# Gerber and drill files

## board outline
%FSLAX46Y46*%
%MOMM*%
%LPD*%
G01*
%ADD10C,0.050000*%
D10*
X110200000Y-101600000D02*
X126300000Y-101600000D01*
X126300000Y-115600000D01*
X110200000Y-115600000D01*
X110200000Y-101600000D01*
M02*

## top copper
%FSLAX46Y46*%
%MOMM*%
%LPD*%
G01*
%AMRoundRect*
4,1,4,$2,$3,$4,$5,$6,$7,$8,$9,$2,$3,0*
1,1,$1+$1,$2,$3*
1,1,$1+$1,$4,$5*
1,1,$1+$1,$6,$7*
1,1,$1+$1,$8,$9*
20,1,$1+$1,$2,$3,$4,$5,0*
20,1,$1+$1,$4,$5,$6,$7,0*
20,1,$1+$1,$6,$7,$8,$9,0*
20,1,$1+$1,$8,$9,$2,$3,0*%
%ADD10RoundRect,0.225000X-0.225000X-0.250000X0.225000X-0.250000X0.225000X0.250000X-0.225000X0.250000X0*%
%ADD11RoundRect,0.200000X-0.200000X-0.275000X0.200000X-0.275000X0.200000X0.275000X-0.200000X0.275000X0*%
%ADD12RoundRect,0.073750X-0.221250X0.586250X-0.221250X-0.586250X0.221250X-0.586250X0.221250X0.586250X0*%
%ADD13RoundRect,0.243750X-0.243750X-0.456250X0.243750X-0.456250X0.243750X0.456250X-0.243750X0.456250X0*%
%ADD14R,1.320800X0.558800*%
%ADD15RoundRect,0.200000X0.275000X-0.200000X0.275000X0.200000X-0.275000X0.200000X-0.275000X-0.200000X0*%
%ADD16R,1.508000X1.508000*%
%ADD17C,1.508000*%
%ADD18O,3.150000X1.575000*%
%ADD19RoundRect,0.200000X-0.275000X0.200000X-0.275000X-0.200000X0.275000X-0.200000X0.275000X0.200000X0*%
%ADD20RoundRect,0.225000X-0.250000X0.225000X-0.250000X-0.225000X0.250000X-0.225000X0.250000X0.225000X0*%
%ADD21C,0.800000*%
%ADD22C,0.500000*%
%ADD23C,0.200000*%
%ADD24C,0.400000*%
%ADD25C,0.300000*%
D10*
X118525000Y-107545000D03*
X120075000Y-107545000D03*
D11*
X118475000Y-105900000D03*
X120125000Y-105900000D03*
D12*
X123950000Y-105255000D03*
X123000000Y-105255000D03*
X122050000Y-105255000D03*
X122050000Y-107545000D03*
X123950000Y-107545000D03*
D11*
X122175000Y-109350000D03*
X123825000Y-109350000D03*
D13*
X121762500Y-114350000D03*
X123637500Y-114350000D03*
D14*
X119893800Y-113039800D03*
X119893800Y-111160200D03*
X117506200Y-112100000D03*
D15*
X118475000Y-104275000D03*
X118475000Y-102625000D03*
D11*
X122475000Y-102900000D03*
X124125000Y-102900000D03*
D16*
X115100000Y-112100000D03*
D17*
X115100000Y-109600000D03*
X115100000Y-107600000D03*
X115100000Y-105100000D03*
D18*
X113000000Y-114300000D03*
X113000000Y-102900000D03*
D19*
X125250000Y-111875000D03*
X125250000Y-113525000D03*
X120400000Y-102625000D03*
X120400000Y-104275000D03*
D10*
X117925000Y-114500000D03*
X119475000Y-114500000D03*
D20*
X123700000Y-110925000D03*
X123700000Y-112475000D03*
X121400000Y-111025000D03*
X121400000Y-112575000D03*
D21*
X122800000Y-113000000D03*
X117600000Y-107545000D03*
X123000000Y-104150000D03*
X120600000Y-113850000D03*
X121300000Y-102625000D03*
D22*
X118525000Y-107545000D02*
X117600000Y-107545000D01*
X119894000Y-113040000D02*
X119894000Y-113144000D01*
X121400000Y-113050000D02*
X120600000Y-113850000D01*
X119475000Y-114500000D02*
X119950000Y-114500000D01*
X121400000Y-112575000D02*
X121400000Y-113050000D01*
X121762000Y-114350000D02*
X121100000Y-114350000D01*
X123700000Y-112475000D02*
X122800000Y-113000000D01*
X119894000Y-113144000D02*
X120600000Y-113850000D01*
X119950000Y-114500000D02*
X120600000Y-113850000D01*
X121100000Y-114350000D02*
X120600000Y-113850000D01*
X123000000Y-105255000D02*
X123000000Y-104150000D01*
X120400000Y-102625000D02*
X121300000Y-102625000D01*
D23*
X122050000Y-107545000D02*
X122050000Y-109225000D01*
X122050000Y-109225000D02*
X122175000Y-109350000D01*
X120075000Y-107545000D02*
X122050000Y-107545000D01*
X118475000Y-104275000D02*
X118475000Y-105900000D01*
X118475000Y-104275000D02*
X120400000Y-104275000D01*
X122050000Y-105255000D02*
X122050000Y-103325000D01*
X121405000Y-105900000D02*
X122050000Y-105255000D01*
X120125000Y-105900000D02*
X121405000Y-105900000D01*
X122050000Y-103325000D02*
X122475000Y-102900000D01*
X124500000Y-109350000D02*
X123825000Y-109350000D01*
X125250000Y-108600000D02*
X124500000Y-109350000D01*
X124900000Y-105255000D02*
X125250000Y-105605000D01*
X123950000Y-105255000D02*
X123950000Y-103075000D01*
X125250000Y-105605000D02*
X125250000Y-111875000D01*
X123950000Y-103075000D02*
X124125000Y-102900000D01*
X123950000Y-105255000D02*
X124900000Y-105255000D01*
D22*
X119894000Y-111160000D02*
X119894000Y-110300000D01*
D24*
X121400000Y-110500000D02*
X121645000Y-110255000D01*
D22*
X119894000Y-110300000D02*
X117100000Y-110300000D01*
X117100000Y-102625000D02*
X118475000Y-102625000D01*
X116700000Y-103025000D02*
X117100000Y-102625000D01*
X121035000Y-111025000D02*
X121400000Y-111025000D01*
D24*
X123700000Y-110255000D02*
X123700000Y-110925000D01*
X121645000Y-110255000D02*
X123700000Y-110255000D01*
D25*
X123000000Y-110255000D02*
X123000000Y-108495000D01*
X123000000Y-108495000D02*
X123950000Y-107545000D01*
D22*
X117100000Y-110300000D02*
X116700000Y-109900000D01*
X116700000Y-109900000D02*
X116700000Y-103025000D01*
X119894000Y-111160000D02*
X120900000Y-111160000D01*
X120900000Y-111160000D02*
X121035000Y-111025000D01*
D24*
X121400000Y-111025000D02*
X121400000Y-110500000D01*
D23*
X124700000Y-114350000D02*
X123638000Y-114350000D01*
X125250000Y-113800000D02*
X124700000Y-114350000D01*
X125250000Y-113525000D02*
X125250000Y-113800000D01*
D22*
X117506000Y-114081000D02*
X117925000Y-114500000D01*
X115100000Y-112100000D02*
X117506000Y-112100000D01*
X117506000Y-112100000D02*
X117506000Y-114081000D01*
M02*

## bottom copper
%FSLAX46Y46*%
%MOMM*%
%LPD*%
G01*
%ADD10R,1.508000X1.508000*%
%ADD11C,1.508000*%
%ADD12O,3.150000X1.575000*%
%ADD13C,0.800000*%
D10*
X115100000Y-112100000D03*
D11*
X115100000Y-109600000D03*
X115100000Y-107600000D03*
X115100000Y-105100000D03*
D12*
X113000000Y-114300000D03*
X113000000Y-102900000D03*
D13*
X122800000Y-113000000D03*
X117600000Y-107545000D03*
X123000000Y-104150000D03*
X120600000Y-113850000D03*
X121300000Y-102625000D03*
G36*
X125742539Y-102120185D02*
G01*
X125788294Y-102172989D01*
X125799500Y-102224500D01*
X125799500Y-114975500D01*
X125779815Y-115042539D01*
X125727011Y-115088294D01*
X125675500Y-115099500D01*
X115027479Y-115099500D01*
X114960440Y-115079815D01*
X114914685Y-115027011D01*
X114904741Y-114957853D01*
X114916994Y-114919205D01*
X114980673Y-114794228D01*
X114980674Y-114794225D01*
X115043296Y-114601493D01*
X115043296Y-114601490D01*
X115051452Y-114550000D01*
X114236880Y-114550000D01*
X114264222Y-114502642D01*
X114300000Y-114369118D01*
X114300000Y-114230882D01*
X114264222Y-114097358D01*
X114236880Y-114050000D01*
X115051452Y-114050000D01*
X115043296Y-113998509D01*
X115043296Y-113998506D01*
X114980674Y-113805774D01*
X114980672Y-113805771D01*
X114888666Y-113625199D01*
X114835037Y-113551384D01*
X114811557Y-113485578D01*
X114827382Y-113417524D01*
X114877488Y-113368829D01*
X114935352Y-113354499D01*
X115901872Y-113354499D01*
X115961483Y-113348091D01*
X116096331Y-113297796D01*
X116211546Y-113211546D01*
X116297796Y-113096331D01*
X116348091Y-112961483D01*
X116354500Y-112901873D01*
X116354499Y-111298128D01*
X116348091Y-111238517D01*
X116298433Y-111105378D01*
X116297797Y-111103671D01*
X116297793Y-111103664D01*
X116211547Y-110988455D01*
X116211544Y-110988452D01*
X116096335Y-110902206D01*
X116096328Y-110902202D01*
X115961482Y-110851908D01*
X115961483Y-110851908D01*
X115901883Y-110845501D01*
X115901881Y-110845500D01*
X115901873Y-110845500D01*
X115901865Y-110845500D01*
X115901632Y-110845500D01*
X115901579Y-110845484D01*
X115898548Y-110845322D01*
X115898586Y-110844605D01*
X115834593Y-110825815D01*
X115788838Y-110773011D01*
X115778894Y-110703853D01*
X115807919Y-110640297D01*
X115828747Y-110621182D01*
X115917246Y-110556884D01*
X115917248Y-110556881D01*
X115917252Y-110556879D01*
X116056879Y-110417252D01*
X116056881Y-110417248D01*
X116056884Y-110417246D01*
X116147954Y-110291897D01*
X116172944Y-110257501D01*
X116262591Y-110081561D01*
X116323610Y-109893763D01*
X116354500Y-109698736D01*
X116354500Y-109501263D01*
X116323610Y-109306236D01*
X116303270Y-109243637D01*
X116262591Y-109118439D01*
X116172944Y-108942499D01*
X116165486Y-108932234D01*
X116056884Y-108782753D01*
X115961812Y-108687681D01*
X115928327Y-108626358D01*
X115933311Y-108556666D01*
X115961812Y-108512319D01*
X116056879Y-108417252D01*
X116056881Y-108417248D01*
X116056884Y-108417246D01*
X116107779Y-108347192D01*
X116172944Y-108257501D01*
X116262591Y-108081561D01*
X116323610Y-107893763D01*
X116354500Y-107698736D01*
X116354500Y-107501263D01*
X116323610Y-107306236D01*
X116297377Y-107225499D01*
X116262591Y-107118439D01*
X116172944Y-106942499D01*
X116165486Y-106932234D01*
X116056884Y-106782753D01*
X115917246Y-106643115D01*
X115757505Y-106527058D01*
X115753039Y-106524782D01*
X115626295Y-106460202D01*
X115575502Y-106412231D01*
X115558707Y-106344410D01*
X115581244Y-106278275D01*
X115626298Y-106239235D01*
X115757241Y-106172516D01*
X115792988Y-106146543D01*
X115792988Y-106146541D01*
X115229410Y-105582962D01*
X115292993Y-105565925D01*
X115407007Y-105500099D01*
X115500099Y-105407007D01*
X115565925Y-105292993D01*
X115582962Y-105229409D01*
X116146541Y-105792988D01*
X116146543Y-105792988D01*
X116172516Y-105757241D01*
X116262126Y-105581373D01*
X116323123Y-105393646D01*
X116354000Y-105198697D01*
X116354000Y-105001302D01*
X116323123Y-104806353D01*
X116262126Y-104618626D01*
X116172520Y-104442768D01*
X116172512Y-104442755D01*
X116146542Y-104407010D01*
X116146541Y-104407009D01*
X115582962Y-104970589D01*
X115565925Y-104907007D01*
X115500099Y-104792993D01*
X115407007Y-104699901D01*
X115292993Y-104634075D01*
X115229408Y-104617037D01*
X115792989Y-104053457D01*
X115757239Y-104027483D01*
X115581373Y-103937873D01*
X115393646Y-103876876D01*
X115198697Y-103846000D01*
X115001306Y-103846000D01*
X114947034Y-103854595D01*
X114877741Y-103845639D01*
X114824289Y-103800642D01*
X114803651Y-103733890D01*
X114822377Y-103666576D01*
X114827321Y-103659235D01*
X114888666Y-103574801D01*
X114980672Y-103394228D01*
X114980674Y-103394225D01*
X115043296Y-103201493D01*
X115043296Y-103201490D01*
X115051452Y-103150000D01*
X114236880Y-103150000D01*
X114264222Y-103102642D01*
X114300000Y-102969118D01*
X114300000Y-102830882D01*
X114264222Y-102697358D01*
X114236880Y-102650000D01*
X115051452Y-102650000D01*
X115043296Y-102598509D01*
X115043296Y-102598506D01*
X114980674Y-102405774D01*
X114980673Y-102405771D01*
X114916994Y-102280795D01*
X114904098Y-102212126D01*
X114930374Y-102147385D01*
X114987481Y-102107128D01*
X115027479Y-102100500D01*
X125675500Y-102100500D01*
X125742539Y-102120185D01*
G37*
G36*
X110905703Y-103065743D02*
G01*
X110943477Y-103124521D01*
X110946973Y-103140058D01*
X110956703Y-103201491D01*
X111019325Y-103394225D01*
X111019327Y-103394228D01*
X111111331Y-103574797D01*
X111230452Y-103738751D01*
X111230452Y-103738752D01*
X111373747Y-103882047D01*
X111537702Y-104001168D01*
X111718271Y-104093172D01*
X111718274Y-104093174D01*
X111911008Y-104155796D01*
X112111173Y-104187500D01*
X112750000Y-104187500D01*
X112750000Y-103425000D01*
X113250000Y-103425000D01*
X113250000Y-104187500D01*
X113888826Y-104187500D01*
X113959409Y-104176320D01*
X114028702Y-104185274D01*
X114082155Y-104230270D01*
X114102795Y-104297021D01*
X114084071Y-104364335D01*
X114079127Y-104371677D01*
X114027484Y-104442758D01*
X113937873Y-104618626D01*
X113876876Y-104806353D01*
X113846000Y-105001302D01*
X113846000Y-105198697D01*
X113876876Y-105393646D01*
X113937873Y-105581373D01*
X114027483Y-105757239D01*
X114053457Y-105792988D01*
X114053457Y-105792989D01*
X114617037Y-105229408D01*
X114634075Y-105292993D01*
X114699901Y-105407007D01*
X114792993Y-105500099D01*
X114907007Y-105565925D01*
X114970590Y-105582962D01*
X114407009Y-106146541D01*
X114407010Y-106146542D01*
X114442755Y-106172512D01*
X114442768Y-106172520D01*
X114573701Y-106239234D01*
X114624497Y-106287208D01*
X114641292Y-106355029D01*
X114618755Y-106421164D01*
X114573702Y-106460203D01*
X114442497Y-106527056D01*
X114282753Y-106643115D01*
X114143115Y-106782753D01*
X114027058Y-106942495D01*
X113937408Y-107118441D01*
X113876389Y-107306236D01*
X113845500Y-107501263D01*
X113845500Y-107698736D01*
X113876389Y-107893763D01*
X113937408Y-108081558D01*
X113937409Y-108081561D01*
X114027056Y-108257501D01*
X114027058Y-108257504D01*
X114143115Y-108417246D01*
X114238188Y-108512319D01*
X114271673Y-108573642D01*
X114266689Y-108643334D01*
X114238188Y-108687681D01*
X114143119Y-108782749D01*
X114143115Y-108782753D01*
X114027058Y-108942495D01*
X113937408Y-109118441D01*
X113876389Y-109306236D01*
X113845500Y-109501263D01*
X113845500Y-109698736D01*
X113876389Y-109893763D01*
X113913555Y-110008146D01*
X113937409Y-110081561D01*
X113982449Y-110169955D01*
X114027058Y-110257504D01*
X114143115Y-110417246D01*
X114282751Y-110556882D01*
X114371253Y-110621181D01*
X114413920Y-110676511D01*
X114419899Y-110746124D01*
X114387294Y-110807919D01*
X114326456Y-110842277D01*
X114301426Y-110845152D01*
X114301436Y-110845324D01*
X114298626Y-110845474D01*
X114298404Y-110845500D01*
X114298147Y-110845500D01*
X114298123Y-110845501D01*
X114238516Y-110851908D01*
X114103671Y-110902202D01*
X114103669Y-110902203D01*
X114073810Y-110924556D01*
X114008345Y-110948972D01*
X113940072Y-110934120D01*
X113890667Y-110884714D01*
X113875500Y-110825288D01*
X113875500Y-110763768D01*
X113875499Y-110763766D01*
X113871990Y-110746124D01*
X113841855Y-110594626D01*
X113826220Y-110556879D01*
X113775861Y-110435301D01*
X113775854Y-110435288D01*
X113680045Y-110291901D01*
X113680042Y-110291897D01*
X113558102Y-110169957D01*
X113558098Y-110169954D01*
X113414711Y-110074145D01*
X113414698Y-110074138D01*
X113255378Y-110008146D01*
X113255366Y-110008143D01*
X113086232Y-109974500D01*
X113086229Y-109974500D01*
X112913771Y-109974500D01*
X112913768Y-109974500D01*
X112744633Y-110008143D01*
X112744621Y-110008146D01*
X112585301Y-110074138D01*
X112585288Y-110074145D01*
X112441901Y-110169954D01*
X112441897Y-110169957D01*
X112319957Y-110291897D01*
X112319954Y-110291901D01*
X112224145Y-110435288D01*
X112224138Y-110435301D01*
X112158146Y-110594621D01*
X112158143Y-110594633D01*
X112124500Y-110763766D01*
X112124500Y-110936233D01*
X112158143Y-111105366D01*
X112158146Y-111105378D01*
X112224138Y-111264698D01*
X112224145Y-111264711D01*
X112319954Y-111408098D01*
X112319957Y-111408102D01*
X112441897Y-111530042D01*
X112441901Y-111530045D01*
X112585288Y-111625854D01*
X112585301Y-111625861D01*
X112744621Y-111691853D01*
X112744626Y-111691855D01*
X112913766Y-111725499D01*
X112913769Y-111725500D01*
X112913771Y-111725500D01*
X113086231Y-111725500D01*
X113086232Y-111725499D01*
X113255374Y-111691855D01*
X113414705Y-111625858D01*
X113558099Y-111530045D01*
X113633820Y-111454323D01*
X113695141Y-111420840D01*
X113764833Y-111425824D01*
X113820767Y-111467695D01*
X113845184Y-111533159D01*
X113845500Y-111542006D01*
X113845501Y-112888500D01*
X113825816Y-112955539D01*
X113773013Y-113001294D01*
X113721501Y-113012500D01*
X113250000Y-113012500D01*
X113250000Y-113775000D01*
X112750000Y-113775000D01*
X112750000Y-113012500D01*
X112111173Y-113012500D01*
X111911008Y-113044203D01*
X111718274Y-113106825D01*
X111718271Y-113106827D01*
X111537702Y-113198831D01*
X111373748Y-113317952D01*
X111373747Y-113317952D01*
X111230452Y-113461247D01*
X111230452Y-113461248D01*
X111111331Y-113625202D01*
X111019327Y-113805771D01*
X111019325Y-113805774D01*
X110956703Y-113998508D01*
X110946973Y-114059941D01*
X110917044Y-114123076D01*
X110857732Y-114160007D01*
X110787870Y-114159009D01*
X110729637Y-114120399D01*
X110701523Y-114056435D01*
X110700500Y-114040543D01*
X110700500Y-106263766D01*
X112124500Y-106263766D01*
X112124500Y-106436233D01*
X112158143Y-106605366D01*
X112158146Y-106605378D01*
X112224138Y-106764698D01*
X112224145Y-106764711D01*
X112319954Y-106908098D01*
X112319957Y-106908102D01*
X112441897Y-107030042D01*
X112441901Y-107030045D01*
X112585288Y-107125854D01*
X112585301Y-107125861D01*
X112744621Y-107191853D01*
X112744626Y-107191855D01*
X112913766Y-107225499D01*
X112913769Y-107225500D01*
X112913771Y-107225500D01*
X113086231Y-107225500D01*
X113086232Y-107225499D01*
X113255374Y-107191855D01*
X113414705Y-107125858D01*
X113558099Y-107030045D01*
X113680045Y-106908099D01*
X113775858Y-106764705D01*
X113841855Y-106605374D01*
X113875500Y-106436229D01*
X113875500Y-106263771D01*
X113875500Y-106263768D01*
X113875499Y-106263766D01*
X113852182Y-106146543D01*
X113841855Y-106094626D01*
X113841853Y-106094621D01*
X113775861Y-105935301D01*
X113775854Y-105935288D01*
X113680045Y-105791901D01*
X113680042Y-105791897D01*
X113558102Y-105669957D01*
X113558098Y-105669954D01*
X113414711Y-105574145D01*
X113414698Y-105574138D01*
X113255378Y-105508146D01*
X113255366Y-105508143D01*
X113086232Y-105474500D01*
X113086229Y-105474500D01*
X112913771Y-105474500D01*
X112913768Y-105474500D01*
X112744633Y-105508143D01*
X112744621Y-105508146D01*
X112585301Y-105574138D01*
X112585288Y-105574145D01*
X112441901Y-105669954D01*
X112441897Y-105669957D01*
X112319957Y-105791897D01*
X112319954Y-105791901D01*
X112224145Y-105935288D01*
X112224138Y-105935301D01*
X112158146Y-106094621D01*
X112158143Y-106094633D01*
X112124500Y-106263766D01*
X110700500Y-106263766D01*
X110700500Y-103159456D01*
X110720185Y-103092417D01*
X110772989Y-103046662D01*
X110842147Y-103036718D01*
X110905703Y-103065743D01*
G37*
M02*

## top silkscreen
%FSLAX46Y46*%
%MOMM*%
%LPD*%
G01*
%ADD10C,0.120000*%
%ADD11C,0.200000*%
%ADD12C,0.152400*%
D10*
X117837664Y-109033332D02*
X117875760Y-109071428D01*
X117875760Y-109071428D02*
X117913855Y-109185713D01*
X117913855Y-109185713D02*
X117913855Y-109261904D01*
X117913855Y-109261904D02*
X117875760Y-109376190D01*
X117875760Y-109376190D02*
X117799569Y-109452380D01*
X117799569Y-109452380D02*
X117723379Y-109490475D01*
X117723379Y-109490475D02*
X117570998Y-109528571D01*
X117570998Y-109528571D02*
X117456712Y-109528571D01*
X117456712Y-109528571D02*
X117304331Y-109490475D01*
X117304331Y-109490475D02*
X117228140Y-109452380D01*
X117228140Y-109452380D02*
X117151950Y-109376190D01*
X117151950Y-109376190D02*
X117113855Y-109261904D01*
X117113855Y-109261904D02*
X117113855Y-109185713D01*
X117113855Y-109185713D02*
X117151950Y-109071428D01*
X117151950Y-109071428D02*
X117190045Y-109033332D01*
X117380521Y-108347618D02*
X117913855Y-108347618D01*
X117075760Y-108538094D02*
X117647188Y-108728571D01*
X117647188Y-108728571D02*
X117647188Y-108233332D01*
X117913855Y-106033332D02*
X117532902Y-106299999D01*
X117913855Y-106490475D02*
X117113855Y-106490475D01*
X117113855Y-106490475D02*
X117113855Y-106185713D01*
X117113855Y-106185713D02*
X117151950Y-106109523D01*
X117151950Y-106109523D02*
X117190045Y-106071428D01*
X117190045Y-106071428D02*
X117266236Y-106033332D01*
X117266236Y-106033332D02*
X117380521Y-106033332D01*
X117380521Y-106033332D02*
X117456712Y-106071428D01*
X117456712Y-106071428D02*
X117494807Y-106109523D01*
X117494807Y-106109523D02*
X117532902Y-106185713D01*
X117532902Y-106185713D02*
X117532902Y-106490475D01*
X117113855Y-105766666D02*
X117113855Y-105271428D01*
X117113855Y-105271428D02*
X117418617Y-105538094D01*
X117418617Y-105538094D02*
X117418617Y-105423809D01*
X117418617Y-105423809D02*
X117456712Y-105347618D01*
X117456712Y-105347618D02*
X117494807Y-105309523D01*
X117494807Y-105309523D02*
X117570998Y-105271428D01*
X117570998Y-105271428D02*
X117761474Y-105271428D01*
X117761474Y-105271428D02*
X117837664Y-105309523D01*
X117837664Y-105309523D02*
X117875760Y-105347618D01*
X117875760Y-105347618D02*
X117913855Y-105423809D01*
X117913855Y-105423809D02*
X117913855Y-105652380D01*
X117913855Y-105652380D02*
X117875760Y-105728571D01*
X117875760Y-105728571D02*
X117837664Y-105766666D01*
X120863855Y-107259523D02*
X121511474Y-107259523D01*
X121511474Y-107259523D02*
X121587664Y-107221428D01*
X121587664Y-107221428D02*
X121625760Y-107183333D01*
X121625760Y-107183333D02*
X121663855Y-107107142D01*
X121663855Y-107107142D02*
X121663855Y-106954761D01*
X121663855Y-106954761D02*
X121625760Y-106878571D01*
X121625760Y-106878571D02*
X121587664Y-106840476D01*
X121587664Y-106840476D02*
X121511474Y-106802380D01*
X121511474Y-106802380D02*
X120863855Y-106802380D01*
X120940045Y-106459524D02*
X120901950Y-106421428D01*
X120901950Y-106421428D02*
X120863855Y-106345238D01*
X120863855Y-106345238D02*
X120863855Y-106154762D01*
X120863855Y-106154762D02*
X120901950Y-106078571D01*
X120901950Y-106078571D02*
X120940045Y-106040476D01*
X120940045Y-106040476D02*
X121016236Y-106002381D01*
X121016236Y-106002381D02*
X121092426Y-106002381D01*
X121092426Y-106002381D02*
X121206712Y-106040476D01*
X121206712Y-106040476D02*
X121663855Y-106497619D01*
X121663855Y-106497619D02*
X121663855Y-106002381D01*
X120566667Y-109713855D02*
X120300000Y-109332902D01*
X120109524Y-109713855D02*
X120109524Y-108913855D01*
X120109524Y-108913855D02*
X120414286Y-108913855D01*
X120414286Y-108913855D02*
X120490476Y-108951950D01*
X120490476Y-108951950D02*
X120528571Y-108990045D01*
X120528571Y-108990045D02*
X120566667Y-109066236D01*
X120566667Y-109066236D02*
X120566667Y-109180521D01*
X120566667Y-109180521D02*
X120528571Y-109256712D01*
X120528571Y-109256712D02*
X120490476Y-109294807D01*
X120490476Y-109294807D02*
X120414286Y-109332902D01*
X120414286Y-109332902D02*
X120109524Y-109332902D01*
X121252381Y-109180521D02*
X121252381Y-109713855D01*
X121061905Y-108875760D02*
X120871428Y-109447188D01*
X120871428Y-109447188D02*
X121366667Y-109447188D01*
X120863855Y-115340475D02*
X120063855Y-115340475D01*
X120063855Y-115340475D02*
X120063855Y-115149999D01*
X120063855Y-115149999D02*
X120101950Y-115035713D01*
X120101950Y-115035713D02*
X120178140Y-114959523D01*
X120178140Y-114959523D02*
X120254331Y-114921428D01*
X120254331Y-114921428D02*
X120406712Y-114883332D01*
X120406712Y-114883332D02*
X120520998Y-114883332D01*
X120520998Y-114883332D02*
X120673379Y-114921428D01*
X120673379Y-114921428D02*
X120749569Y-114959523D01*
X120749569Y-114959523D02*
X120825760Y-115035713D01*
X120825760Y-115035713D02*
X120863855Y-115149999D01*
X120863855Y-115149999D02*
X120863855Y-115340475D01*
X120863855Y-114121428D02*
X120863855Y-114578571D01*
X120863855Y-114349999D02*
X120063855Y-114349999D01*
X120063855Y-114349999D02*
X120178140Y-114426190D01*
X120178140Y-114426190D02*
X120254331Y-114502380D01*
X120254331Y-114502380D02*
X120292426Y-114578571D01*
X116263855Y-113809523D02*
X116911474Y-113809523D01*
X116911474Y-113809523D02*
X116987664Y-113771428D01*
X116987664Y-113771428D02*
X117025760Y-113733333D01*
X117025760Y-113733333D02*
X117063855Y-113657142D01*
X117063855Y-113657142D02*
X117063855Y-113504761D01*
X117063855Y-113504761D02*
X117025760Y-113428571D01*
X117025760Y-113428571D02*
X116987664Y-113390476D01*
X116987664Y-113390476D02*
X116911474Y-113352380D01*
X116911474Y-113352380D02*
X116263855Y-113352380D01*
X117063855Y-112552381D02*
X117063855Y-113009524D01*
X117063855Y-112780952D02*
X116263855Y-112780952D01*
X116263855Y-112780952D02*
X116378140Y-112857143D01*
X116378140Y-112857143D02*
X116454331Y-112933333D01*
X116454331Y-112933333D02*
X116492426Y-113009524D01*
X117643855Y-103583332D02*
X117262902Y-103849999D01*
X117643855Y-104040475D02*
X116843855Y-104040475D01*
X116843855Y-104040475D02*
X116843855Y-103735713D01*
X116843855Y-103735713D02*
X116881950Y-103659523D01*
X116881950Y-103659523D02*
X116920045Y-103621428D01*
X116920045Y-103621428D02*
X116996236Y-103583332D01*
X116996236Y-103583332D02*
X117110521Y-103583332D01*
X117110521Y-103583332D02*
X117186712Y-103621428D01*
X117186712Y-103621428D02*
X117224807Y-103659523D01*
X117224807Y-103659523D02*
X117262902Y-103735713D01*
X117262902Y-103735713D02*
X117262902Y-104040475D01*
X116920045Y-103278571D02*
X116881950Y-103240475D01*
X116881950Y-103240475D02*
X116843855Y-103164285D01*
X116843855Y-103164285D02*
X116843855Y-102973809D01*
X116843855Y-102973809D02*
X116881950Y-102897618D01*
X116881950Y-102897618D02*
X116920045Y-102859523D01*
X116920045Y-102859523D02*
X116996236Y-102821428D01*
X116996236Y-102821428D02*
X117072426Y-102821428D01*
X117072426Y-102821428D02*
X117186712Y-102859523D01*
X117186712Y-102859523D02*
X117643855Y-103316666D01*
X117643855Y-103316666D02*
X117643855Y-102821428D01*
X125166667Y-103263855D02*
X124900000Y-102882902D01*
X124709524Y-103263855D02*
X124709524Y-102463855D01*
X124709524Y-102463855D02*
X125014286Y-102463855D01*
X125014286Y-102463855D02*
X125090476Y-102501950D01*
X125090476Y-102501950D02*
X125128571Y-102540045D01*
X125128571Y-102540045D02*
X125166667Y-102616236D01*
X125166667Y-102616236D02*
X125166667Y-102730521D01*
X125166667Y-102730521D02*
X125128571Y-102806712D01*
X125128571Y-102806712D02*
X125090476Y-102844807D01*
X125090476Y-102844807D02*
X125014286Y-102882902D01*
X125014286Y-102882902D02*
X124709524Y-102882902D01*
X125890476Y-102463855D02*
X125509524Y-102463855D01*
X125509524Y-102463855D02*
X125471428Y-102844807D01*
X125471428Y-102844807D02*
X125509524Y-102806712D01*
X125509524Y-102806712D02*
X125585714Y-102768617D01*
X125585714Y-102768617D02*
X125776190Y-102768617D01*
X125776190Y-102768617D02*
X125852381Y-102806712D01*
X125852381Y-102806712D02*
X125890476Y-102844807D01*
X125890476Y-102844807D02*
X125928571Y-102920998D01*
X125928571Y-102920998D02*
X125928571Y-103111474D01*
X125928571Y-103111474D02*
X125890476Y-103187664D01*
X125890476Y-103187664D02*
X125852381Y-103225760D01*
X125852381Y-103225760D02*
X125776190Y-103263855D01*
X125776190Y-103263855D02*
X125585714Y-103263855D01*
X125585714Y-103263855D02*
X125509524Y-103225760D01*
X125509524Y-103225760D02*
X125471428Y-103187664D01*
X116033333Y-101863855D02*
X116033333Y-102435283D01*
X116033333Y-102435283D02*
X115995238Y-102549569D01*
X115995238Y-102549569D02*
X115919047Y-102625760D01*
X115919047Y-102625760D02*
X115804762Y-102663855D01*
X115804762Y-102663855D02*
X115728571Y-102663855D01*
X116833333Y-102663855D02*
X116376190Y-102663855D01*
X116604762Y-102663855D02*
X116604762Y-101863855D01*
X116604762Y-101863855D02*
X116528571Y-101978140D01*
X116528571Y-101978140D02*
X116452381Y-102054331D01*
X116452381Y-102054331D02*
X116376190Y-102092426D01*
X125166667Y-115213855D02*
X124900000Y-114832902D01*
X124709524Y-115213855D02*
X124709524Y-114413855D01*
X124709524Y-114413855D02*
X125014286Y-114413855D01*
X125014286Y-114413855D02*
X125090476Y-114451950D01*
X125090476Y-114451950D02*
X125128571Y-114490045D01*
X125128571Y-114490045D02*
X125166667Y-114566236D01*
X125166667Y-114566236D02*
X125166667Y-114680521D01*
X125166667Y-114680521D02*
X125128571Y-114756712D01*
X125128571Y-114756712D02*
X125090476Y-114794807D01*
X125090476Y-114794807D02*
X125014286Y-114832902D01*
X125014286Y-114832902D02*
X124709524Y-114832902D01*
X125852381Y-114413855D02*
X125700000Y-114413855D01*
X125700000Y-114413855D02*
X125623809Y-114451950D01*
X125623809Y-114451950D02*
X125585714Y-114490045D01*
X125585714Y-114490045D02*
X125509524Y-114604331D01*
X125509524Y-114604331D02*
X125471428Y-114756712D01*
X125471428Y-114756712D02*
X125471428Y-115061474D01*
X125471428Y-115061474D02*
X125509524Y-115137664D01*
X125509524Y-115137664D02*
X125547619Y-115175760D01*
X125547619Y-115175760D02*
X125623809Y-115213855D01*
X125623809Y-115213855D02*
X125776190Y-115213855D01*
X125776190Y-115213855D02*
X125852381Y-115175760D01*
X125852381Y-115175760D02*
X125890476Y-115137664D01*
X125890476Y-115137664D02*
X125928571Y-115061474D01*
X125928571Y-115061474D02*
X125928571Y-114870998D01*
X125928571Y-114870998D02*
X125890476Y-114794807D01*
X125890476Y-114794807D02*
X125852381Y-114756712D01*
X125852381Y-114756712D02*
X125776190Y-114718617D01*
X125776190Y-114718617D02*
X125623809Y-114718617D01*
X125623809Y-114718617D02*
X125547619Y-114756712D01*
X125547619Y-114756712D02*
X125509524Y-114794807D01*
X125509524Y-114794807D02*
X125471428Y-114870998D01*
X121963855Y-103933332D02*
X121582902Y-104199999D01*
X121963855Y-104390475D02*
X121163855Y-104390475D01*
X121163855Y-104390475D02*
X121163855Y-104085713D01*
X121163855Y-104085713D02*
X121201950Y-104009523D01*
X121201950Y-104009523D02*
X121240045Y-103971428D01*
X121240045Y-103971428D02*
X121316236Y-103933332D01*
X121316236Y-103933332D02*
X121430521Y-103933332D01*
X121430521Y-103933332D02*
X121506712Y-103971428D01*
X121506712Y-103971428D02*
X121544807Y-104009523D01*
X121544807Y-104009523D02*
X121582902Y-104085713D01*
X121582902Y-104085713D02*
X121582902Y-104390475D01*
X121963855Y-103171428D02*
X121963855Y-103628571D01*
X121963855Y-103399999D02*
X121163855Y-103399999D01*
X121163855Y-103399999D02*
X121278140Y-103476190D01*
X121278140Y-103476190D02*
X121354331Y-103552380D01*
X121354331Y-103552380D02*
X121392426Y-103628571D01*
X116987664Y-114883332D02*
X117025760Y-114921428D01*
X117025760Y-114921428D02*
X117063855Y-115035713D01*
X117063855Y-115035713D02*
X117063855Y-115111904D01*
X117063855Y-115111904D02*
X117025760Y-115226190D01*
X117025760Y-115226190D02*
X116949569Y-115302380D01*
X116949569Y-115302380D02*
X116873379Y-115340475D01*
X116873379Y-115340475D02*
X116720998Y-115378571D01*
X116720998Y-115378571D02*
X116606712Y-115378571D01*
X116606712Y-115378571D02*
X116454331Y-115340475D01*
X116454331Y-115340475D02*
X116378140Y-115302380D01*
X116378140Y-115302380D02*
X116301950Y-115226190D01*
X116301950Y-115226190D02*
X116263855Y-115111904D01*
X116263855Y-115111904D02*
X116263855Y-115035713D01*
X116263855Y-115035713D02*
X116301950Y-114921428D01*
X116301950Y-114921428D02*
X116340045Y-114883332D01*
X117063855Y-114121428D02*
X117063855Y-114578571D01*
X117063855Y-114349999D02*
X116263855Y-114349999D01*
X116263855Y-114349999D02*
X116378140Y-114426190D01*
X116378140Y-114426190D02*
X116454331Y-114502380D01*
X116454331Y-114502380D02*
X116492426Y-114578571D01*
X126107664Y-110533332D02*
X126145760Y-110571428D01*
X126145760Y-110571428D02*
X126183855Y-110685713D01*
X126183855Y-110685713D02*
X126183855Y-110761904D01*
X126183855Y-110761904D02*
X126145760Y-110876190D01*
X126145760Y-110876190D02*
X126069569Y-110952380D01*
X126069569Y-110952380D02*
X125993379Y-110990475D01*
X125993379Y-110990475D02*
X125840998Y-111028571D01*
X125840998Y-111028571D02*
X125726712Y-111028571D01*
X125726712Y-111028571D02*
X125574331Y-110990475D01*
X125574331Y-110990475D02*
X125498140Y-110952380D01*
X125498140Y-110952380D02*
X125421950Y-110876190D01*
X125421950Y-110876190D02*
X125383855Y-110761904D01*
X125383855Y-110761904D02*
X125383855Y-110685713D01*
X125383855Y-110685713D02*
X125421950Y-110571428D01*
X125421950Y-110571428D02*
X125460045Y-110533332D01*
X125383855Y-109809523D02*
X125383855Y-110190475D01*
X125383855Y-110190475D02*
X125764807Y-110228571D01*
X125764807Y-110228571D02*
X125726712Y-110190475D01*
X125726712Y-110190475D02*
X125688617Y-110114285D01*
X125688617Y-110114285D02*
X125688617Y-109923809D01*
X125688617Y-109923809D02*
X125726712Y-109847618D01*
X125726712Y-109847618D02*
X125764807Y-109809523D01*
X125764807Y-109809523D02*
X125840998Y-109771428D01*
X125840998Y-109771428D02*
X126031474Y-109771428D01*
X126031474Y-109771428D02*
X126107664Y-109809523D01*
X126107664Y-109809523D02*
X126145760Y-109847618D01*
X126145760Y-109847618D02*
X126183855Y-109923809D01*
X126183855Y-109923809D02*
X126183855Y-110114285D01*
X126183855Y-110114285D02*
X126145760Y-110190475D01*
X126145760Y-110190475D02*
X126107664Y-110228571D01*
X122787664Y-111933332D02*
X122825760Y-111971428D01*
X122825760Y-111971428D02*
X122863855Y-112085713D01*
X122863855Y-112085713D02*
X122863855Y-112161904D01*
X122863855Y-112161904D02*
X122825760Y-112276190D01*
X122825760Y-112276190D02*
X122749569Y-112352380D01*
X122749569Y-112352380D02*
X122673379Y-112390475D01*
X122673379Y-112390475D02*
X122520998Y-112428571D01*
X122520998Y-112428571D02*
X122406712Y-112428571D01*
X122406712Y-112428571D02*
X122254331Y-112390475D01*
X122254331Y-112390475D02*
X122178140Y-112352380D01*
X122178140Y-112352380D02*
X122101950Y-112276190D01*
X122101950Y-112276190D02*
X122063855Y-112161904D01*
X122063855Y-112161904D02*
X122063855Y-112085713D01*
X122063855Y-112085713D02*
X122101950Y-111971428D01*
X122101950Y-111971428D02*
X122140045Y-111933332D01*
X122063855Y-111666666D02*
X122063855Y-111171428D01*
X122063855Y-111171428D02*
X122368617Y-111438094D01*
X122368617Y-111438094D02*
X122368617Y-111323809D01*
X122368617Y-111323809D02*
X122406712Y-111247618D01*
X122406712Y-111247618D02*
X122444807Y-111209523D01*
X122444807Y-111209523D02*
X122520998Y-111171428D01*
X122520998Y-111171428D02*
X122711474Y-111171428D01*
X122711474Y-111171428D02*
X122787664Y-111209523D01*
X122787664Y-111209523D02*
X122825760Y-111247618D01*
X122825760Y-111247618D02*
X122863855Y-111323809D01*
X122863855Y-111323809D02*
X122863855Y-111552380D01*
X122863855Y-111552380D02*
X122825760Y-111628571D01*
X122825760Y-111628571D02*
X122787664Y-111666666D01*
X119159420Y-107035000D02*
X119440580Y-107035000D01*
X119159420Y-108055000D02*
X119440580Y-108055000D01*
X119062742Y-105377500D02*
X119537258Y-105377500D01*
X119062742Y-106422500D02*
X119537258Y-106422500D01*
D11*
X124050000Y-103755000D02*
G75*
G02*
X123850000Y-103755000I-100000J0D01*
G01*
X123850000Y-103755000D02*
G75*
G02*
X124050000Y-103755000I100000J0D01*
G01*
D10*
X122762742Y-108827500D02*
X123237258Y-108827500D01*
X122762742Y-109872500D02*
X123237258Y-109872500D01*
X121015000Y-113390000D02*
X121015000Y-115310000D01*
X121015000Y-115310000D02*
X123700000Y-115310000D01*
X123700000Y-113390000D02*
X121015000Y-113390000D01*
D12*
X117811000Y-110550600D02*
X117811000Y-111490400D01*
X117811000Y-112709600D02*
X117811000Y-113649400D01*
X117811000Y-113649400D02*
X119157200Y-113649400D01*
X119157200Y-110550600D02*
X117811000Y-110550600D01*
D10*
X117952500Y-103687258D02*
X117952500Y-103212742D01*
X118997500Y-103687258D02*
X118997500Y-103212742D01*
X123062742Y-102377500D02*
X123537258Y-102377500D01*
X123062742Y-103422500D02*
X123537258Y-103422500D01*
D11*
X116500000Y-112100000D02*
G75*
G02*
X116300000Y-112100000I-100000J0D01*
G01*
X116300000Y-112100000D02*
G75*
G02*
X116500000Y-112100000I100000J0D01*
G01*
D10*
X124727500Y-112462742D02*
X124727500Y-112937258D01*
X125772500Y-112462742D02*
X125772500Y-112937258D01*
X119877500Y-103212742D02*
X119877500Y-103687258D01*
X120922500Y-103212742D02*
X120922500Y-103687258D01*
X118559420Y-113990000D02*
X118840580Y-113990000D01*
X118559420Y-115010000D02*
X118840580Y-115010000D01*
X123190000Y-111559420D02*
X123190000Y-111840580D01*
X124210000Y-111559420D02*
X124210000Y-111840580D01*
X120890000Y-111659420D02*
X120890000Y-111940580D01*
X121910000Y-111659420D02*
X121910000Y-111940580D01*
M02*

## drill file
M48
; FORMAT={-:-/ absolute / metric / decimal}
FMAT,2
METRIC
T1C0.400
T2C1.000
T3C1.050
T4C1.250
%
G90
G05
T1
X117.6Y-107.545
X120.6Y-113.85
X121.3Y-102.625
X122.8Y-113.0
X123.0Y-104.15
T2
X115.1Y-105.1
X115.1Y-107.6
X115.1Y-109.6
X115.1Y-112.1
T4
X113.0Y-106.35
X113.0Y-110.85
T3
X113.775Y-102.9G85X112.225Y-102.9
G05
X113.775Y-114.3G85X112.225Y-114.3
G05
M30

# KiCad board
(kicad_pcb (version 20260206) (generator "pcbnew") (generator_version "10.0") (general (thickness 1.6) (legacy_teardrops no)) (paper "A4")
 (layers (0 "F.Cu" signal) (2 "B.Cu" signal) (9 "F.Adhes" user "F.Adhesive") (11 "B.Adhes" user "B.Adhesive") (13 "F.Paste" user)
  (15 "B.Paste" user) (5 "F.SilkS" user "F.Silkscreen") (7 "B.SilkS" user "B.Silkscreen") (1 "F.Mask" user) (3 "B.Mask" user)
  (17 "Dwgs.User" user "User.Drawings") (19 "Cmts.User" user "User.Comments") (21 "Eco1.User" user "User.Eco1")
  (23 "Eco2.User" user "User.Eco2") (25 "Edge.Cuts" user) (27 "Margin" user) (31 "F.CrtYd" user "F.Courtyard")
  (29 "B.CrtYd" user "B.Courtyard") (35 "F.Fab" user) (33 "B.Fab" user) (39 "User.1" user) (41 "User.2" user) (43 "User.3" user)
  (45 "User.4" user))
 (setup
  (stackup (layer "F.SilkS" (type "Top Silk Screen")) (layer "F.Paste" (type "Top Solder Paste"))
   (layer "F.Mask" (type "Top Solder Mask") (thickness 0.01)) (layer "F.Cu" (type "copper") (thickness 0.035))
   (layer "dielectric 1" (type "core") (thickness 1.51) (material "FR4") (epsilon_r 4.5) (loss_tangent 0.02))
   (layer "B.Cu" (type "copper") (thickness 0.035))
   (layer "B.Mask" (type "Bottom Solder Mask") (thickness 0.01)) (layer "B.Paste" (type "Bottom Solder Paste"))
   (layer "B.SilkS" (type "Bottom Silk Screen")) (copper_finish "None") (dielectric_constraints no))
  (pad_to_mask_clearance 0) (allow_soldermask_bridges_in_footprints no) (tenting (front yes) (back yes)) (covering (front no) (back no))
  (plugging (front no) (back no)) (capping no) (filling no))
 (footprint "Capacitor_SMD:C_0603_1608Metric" (layer "F.Cu") (at 119.3 107.545)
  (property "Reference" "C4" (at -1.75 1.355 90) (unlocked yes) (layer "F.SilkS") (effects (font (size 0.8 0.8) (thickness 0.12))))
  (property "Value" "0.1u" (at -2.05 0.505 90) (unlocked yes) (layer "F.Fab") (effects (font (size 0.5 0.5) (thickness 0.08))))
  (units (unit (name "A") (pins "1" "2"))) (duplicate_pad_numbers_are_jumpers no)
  (fp_line (start -0.14058 -0.51) (end 0.14058 -0.51) (stroke (width 0.12) (type solid)) (layer "F.SilkS"))
  (fp_line (start -0.14058 0.51) (end 0.14058 0.51) (stroke (width 0.12) (type solid)) (layer "F.SilkS"))
  (pad "1" smd roundrect (at -0.775 0) (size 0.9 0.95) (layers "F.Cu" "F.Mask" "F.Paste") (roundrect_rratio 0.25) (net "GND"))
  (pad "2" smd roundrect (at 0.775 0) (size 0.9 0.95) (layers "F.Cu" "F.Mask" "F.Paste") (roundrect_rratio 0.25) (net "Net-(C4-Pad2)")))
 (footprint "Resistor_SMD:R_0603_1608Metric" (layer "F.Cu") (at 119.3 105.9)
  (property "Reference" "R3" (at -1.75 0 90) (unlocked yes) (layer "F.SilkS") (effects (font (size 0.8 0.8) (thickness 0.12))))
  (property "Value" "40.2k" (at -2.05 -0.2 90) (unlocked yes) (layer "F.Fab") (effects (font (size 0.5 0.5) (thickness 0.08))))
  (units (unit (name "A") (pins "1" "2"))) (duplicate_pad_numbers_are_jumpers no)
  (fp_line (start -0.237258 -0.5225) (end 0.237258 -0.5225) (stroke (width 0.12) (type solid)) (layer "F.SilkS"))
  (fp_line (start -0.237258 0.5225) (end 0.237258 0.5225) (stroke (width 0.12) (type solid)) (layer "F.SilkS"))
  (pad "1" smd roundrect (at -0.825 0) (size 0.8 0.95) (layers "F.Cu" "F.Mask" "F.Paste") (roundrect_rratio 0.25) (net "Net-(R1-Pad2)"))
  (pad "2" smd roundrect (at 0.825 0) (size 0.8 0.95) (layers "F.Cu" "F.Mask" "F.Paste") (roundrect_rratio 0.25) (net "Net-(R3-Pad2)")))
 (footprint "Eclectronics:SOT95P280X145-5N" (layer "F.Cu") (at 123 106.4 -90)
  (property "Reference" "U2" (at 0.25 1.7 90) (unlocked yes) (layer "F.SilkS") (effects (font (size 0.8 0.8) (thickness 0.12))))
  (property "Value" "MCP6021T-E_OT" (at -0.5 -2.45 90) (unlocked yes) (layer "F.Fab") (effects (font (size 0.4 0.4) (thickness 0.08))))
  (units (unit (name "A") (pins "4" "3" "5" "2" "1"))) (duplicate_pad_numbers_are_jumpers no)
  (fp_circle (center -2.645 -0.95) (end -2.545 -0.95) (stroke (width 0.2) (type solid)) (fill no) (layer "F.SilkS"))
  (pad "1" smd roundrect (at -1.145 -0.95 270) (size 1.32 0.59) (layers "F.Cu" "F.Mask" "F.Paste") (roundrect_rratio 0.125)
   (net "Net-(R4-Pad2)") (solder_mask_margin 0.102))
  (pad "2" smd roundrect (at -1.145 0 270) (size 1.32 0.59) (layers "F.Cu" "F.Mask" "F.Paste") (roundrect_rratio 0.125) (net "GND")
   (solder_mask_margin 0.102))
  (pad "3" smd roundrect (at -1.145 0.95 270) (size 1.32 0.59) (layers "F.Cu" "F.Mask" "F.Paste") (roundrect_rratio 0.125)
   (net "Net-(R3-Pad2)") (solder_mask_margin 0.102))
  (pad "4" smd roundrect (at 1.145 0.95 270) (size 1.32 0.59) (layers "F.Cu" "F.Mask" "F.Paste") (roundrect_rratio 0.125)
   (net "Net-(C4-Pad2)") (solder_mask_margin 0.102))
  (pad "5" smd roundrect (at 1.145 -0.95 270) (size 1.32 0.59) (layers "F.Cu" "F.Mask" "F.Paste") (roundrect_rratio 0.125) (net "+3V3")
   (solder_mask_margin 0.102)))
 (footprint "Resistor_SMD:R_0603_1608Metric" (layer "F.Cu") (at 123 109.35)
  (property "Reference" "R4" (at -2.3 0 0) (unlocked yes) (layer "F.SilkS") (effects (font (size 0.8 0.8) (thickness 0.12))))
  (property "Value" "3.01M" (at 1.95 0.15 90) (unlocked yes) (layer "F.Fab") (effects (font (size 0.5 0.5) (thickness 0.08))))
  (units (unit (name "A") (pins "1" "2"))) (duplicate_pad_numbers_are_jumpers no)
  (fp_line (start -0.237258 -0.5225) (end 0.237258 -0.5225) (stroke (width 0.12) (type solid)) (layer "F.SilkS"))
  (fp_line (start -0.237258 0.5225) (end 0.237258 0.5225) (stroke (width 0.12) (type solid)) (layer "F.SilkS"))
  (pad "1" smd roundrect (at -0.825 0) (size 0.8 0.95) (layers "F.Cu" "F.Mask" "F.Paste") (roundrect_rratio 0.25) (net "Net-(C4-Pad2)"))
  (pad "2" smd roundrect (at 0.825 0) (size 0.8 0.95) (layers "F.Cu" "F.Mask" "F.Paste") (roundrect_rratio 0.25) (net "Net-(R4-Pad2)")))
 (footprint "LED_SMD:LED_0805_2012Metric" (layer "F.Cu") (at 122.7 114.35)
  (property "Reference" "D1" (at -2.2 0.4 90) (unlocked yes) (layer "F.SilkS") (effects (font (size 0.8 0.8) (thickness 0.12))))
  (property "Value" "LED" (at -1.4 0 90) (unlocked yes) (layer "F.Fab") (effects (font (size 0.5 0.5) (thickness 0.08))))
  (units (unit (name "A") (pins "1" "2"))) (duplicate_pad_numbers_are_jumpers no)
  (fp_line (start -1.685 -0.96) (end -1.685 0.96) (stroke (width 0.12) (type solid)) (layer "F.SilkS"))
  (fp_line (start -1.685 0.96) (end 1 0.96) (stroke (width 0.12) (type solid)) (layer "F.SilkS"))
  (fp_line (start 1 -0.96) (end -1.685 -0.96) (stroke (width 0.12) (type solid)) (layer "F.SilkS"))
  (pad "1" smd roundrect (at -0.9375 0) (size 0.975 1.4) (layers "F.Cu" "F.Mask" "F.Paste") (roundrect_rratio 0.25) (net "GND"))
  (pad "2" smd roundrect (at 0.9375 0) (size 0.975 1.4) (layers "F.Cu" "F.Mask" "F.Paste") (roundrect_rratio 0.25) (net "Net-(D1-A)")))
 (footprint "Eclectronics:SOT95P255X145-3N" (layer "F.Cu") (at 118.7 112.1 90)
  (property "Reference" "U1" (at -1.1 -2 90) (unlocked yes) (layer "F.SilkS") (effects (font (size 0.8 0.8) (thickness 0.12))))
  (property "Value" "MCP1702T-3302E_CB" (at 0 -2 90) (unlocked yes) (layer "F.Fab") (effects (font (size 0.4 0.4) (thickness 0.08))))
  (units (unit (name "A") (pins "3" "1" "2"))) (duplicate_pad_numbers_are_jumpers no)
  (fp_line (start 1.5494 -0.889) (end 0.6096 -0.889) (stroke (width 0.1524) (type solid)) (layer "F.SilkS"))
  (fp_line (start -0.6096 -0.889) (end -1.5494 -0.889) (stroke (width 0.1524) (type solid)) (layer "F.SilkS"))
  (fp_line (start -1.5494 -0.889) (end -1.5494 0.4572) (stroke (width 0.1524) (type solid)) (layer "F.SilkS"))
  (fp_line (start 1.5494 0.4572) (end 1.5494 -0.889) (stroke (width 0.1524) (type solid)) (layer "F.SilkS"))
  (pad "1" smd rect (at -0.9398 1.1938 90) (size 0.5588 1.3208) (layers "F.Cu" "F.Mask" "F.Paste") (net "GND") (solder_mask_margin 0.102))
  (pad "2" smd rect (at 0.9398 1.1938 90) (size 0.5588 1.3208) (layers "F.Cu" "F.Mask" "F.Paste") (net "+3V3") (solder_mask_margin 0.102))
  (pad "3" smd rect (at 0 -1.1938 90) (size 0.5588 1.3208) (layers "F.Cu" "F.Mask" "F.Paste") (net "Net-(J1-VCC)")
   (solder_mask_margin 0.102)))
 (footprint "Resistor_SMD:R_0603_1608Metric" (layer "F.Cu") (at 118.475 103.45 90)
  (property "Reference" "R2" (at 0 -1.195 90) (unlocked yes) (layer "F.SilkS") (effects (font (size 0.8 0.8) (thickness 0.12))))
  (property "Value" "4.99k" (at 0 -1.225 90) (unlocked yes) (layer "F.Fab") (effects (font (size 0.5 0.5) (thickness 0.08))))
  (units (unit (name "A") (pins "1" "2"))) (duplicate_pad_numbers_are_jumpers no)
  (fp_line (start -0.237258 -0.5225) (end 0.237258 -0.5225) (stroke (width 0.12) (type solid)) (layer "F.SilkS"))
  (fp_line (start -0.237258 0.5225) (end 0.237258 0.5225) (stroke (width 0.12) (type solid)) (layer "F.SilkS"))
  (pad "1" smd roundrect (at -0.825 0 90) (size 0.8 0.95) (layers "F.Cu" "F.Mask" "F.Paste") (roundrect_rratio 0.25) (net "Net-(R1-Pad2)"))
  (pad "2" smd roundrect (at 0.825 0 90) (size 0.8 0.95) (layers "F.Cu" "F.Mask" "F.Paste") (roundrect_rratio 0.25) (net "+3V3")))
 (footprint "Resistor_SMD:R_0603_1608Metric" (layer "F.Cu") (at 123.3 102.9)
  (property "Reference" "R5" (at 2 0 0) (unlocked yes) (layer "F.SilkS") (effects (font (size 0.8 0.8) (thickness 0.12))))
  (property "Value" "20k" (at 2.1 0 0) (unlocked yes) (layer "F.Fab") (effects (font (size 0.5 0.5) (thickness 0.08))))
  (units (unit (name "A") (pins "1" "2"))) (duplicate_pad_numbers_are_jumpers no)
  (fp_line (start -0.237258 -0.5225) (end 0.237258 -0.5225) (stroke (width 0.12) (type solid)) (layer "F.SilkS"))
  (fp_line (start -0.237258 0.5225) (end 0.237258 0.5225) (stroke (width 0.12) (type solid)) (layer "F.SilkS"))
  (pad "1" smd roundrect (at -0.825 0) (size 0.8 0.95) (layers "F.Cu" "F.Mask" "F.Paste") (roundrect_rratio 0.25) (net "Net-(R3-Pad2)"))
  (pad "2" smd roundrect (at 0.825 0) (size 0.8 0.95) (layers "F.Cu" "F.Mask" "F.Paste") (roundrect_rratio 0.25) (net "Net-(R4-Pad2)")))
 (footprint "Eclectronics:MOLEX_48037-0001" (layer "F.Cu") (at 113 108.6 -90)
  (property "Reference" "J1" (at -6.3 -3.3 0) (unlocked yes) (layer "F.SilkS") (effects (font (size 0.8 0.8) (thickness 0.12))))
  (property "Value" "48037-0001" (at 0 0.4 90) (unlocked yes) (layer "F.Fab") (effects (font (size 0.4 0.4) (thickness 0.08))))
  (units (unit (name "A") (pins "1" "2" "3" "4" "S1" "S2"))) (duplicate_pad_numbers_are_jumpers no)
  (fp_circle (center 3.5 -3.4) (end 3.6 -3.4) (stroke (width 0.2) (type solid)) (fill no) (layer "F.SilkS"))
  (pad "" np_thru_hole circle (at -2.25 0 270) (size 1.25 1.25) (drill 1.25) (layers "*.Cu" "*.Mask"))
  (pad "" np_thru_hole circle (at 2.25 0 270) (size 1.25 1.25) (drill 1.25) (layers "*.Cu" "*.Mask"))
  (pad "1" thru_hole rect (at 3.5 -2.1 270) (size 1.508 1.508) (drill 1) (layers "*.Cu" "*.Mask") (remove_unused_layers no)
   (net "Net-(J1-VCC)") (solder_mask_margin 0.0762))
  (pad "2" thru_hole circle (at 1 -2.1 270) (size 1.508 1.508) (drill 1) (layers "*.Cu" "*.Mask") (remove_unused_layers no)
   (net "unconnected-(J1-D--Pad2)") (solder_mask_margin 0.0762))
  (pad "3" thru_hole circle (at -1 -2.1 270) (size 1.508 1.508) (drill 1) (layers "*.Cu" "*.Mask") (remove_unused_layers no)
   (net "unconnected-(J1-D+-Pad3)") (solder_mask_margin 0.0762))
  (pad "4" thru_hole circle (at -3.5 -2.1 270) (size 1.508 1.508) (drill 1) (layers "*.Cu" "*.Mask") (remove_unused_layers no) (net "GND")
   (solder_mask_margin 0.0762))
  (pad "S1" thru_hole oval (at 5.7 0 270) (size 1.575 3.15) (drill oval 1.05 2.6) (layers "*.Cu" "*.Mask") (remove_unused_layers no)
   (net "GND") (solder_mask_margin 0.0762))
  (pad "S2" thru_hole oval (at -5.7 0 270) (size 1.575 3.15) (drill oval 1.05 2.6) (layers "*.Cu" "*.Mask") (remove_unused_layers no)
   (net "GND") (solder_mask_margin 0.0762)))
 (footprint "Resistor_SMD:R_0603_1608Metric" (layer "F.Cu") (at 125.25 112.7 -90)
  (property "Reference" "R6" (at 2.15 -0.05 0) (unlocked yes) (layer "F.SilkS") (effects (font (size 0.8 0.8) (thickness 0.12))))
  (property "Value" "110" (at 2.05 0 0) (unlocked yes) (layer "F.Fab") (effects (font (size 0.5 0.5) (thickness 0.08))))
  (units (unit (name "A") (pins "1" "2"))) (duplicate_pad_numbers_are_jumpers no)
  (fp_line (start -0.237258 0.5225) (end 0.237258 0.5225) (stroke (width 0.12) (type solid)) (layer "F.SilkS"))
  (fp_line (start -0.237258 -0.5225) (end 0.237258 -0.5225) (stroke (width 0.12) (type solid)) (layer "F.SilkS"))
  (pad "1" smd roundrect (at -0.825 0 270) (size 0.8 0.95) (layers "F.Cu" "F.Mask" "F.Paste") (roundrect_rratio 0.25) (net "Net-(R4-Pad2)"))
  (pad "2" smd roundrect (at 0.825 0 270) (size 0.8 0.95) (layers "F.Cu" "F.Mask" "F.Paste") (roundrect_rratio 0.25) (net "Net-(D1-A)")))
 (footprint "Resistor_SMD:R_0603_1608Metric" (layer "F.Cu") (at 120.4 103.45 -90)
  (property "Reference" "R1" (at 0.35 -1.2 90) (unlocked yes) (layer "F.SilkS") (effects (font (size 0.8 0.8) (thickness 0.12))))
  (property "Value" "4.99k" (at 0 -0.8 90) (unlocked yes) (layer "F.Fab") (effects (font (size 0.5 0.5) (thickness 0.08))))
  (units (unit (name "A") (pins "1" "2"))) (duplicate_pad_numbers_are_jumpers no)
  (fp_line (start -0.237258 0.5225) (end 0.237258 0.5225) (stroke (width 0.12) (type solid)) (layer "F.SilkS"))
  (fp_line (start -0.237258 -0.5225) (end 0.237258 -0.5225) (stroke (width 0.12) (type solid)) (layer "F.SilkS"))
  (pad "1" smd roundrect (at -0.825 0 270) (size 0.8 0.95) (layers "F.Cu" "F.Mask" "F.Paste") (roundrect_rratio 0.25) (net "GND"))
  (pad "2" smd roundrect (at 0.825 0 270) (size 0.8 0.95) (layers "F.Cu" "F.Mask" "F.Paste") (roundrect_rratio 0.25) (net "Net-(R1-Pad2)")))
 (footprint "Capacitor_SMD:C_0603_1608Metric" (layer "F.Cu") (at 118.7 114.5)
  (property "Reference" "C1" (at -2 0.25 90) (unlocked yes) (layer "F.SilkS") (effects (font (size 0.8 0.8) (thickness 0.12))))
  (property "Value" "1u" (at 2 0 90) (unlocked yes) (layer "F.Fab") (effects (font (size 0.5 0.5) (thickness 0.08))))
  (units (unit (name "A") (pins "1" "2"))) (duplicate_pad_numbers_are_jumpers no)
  (fp_line (start -0.14058 -0.51) (end 0.14058 -0.51) (stroke (width 0.12) (type solid)) (layer "F.SilkS"))
  (fp_line (start -0.14058 0.51) (end 0.14058 0.51) (stroke (width 0.12) (type solid)) (layer "F.SilkS"))
  (pad "1" smd roundrect (at -0.775 0) (size 0.9 0.95) (layers "F.Cu" "F.Mask" "F.Paste") (roundrect_rratio 0.25) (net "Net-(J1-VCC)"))
  (pad "2" smd roundrect (at 0.775 0) (size 0.9 0.95) (layers "F.Cu" "F.Mask" "F.Paste") (roundrect_rratio 0.25) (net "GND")))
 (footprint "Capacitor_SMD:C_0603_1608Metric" (layer "F.Cu") (at 123.7 111.7 -90)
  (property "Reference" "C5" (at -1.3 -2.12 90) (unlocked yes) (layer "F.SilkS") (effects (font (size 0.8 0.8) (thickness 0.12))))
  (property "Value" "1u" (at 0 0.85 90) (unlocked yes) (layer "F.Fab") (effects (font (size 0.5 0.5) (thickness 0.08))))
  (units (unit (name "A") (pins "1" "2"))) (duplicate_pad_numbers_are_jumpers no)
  (fp_line (start -0.14058 0.51) (end 0.14058 0.51) (stroke (width 0.12) (type solid)) (layer "F.SilkS"))
  (fp_line (start -0.14058 -0.51) (end 0.14058 -0.51) (stroke (width 0.12) (type solid)) (layer "F.SilkS"))
  (pad "1" smd roundrect (at -0.775 0 270) (size 0.9 0.95) (layers "F.Cu" "F.Mask" "F.Paste") (roundrect_rratio 0.25) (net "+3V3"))
  (pad "2" smd roundrect (at 0.775 0 270) (size 0.9 0.95) (layers "F.Cu" "F.Mask" "F.Paste") (roundrect_rratio 0.25) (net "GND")))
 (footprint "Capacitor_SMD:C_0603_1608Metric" (layer "F.Cu") (at 121.4 111.8 -90)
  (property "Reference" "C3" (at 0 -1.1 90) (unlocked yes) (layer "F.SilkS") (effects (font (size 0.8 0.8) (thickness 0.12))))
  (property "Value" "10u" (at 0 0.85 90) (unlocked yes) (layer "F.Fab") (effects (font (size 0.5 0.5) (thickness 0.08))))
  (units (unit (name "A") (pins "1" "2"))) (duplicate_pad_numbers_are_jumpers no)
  (fp_line (start -0.14058 0.51) (end 0.14058 0.51) (stroke (width 0.12) (type solid)) (layer "F.SilkS"))
  (fp_line (start -0.14058 -0.51) (end 0.14058 -0.51) (stroke (width 0.12) (type solid)) (layer "F.SilkS"))
  (pad "1" smd roundrect (at -0.775 0 270) (size 0.9 0.95) (layers "F.Cu" "F.Mask" "F.Paste") (roundrect_rratio 0.25) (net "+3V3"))
  (pad "2" smd roundrect (at 0.775 0 270) (size 0.9 0.95) (layers "F.Cu" "F.Mask" "F.Paste") (roundrect_rratio 0.25) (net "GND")))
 (gr_rect (start 110.2 101.6) (end 126.3 115.6) (stroke (width 0.05) (type default)) (fill no) (layer "Edge.Cuts"))
 (segment (start 118.525 107.545) (end 117.6 107.545) (width 0.5) (layer "F.Cu") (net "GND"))
 (segment (start 119.894 113.04) (end 119.894 113.144) (width 0.5) (layer "F.Cu") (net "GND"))
 (segment (start 121.4 113.05) (end 120.6 113.85) (width 0.5) (layer "F.Cu") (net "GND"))
 (segment (start 119.475 114.5) (end 119.95 114.5) (width 0.5) (layer "F.Cu") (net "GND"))
 (segment (start 121.4 112.575) (end 121.4 113.05) (width 0.5) (layer "F.Cu") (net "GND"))
 (segment (start 121.762 114.35) (end 121.1 114.35) (width 0.5) (layer "F.Cu") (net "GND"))
 (segment (start 123.7 112.475) (end 122.8 113) (width 0.5) (layer "F.Cu") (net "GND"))
 (segment (start 119.894 113.144) (end 120.6 113.85) (width 0.5) (layer "F.Cu") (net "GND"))
 (segment (start 119.95 114.5) (end 120.6 113.85) (width 0.5) (layer "F.Cu") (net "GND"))
 (segment (start 121.1 114.35) (end 120.6 113.85) (width 0.5) (layer "F.Cu") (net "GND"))
 (segment (start 123 105.255) (end 123 104.15) (width 0.5) (layer "F.Cu") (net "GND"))
 (segment (start 120.4 102.625) (end 121.3 102.625) (width 0.5) (layer "F.Cu") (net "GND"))
 (via (at 122.8 113) (size 0.8) (drill 0.4) (layers "F.Cu" "B.Cu") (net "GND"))
 (via (at 117.6 107.545) (size 0.8) (drill 0.4) (layers "F.Cu" "B.Cu") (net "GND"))
 (via (at 123 104.15) (size 0.8) (drill 0.4) (layers "F.Cu" "B.Cu") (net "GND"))
 (via (at 120.6 113.85) (size 0.8) (drill 0.4) (layers "F.Cu" "B.Cu") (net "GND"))
 (via (at 121.3 102.625) (size 0.8) (drill 0.4) (layers "F.Cu" "B.Cu") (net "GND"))
 (segment (start 122.05 107.545) (end 122.05 109.225) (width 0.2) (layer "F.Cu") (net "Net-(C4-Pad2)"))
 (segment (start 122.05 109.225) (end 122.175 109.35) (width 0.2) (layer "F.Cu") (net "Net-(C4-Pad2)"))
 (segment (start 120.075 107.545) (end 122.05 107.545) (width 0.2) (layer "F.Cu") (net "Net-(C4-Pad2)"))
 (segment (start 118.475 104.275) (end 118.475 105.9) (width 0.2) (layer "F.Cu") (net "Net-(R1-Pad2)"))
 (segment (start 118.475 104.275) (end 120.4 104.275) (width 0.2) (layer "F.Cu") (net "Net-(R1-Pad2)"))
 (segment (start 122.05 105.255) (end 122.05 103.325) (width 0.2) (layer "F.Cu") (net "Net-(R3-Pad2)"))
 (segment (start 121.405 105.9) (end 122.05 105.255) (width 0.2) (layer "F.Cu") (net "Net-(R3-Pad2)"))
 (segment (start 120.125 105.9) (end 121.405 105.9) (width 0.2) (layer "F.Cu") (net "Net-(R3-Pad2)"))
 (segment (start 122.05 103.325) (end 122.475 102.9) (width 0.2) (layer "F.Cu") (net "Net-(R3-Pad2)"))
 (segment (start 124.5 109.35) (end 123.825 109.35) (width 0.2) (layer "F.Cu") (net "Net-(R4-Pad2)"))
 (segment (start 125.25 108.6) (end 124.5 109.35) (width 0.2) (layer "F.Cu") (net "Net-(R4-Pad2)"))
 (segment (start 124.9 105.255) (end 125.25 105.605) (width 0.2) (layer "F.Cu") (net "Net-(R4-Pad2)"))
 (segment (start 123.95 105.255) (end 123.95 103.075) (width 0.2) (layer "F.Cu") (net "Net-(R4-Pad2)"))
 (segment (start 125.25 105.605) (end 125.25 111.875) (width 0.2) (layer "F.Cu") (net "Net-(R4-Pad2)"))
 (segment (start 123.95 103.075) (end 124.125 102.9) (width 0.2) (layer "F.Cu") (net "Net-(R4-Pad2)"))
 (segment (start 123.95 105.255) (end 124.9 105.255) (width 0.2) (layer "F.Cu") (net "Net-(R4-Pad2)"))
 (segment (start 119.894 111.16) (end 119.894 110.3) (width 0.5) (layer "F.Cu") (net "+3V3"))
 (segment (start 121.4 110.5) (end 121.645 110.255) (width 0.4) (layer "F.Cu") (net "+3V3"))
 (segment (start 119.894 110.3) (end 117.1 110.3) (width 0.5) (layer "F.Cu") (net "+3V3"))
 (segment (start 117.1 102.625) (end 118.475 102.625) (width 0.5) (layer "F.Cu") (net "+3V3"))
 (segment (start 116.7 103.025) (end 117.1 102.625) (width 0.5) (layer "F.Cu") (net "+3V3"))
 (segment (start 121.035 111.025) (end 121.4 111.025) (width 0.5) (layer "F.Cu") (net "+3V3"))
 (segment (start 123.7 110.255) (end 123.7 110.925) (width 0.4) (layer "F.Cu") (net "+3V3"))
 (segment (start 121.645 110.255) (end 123.7 110.255) (width 0.4) (layer "F.Cu") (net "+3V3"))
 (segment (start 123 110.255) (end 123 108.495) (width 0.3) (layer "F.Cu") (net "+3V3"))
 (segment (start 123 108.495) (end 123.95 107.545) (width 0.3) (layer "F.Cu") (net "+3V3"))
 (segment (start 117.1 110.3) (end 116.7 109.9) (width 0.5) (layer "F.Cu") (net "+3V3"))
 (segment (start 116.7 109.9) (end 116.7 103.025) (width 0.5) (layer "F.Cu") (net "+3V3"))
 (segment (start 119.894 111.16) (end 120.9 111.16) (width 0.5) (layer "F.Cu") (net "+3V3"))
 (segment (start 120.9 111.16) (end 121.035 111.025) (width 0.5) (layer "F.Cu") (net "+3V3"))
 (segment (start 121.4 111.025) (end 121.4 110.5) (width 0.4) (layer "F.Cu") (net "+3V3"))
 (segment (start 124.7 114.35) (end 123.638 114.35) (width 0.2) (layer "F.Cu") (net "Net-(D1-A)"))
 (segment (start 125.25 113.8) (end 124.7 114.35) (width 0.2) (layer "F.Cu") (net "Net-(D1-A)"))
 (segment (start 125.25 113.525) (end 125.25 113.8) (width 0.2) (layer "F.Cu") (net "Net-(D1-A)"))
 (segment (start 117.506 114.081) (end 117.925 114.5) (width 0.5) (layer "F.Cu") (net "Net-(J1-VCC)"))
 (segment (start 115.1 112.1) (end 117.506 112.1) (width 0.5) (layer "F.Cu") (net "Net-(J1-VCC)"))
 (segment (start 117.506 112.1) (end 117.506 114.081) (width 0.5) (layer "F.Cu") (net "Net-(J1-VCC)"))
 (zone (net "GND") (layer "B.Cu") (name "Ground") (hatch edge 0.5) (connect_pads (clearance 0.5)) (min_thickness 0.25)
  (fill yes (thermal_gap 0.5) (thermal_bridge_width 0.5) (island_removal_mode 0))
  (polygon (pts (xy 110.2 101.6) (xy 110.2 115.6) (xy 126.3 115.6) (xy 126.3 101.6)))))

